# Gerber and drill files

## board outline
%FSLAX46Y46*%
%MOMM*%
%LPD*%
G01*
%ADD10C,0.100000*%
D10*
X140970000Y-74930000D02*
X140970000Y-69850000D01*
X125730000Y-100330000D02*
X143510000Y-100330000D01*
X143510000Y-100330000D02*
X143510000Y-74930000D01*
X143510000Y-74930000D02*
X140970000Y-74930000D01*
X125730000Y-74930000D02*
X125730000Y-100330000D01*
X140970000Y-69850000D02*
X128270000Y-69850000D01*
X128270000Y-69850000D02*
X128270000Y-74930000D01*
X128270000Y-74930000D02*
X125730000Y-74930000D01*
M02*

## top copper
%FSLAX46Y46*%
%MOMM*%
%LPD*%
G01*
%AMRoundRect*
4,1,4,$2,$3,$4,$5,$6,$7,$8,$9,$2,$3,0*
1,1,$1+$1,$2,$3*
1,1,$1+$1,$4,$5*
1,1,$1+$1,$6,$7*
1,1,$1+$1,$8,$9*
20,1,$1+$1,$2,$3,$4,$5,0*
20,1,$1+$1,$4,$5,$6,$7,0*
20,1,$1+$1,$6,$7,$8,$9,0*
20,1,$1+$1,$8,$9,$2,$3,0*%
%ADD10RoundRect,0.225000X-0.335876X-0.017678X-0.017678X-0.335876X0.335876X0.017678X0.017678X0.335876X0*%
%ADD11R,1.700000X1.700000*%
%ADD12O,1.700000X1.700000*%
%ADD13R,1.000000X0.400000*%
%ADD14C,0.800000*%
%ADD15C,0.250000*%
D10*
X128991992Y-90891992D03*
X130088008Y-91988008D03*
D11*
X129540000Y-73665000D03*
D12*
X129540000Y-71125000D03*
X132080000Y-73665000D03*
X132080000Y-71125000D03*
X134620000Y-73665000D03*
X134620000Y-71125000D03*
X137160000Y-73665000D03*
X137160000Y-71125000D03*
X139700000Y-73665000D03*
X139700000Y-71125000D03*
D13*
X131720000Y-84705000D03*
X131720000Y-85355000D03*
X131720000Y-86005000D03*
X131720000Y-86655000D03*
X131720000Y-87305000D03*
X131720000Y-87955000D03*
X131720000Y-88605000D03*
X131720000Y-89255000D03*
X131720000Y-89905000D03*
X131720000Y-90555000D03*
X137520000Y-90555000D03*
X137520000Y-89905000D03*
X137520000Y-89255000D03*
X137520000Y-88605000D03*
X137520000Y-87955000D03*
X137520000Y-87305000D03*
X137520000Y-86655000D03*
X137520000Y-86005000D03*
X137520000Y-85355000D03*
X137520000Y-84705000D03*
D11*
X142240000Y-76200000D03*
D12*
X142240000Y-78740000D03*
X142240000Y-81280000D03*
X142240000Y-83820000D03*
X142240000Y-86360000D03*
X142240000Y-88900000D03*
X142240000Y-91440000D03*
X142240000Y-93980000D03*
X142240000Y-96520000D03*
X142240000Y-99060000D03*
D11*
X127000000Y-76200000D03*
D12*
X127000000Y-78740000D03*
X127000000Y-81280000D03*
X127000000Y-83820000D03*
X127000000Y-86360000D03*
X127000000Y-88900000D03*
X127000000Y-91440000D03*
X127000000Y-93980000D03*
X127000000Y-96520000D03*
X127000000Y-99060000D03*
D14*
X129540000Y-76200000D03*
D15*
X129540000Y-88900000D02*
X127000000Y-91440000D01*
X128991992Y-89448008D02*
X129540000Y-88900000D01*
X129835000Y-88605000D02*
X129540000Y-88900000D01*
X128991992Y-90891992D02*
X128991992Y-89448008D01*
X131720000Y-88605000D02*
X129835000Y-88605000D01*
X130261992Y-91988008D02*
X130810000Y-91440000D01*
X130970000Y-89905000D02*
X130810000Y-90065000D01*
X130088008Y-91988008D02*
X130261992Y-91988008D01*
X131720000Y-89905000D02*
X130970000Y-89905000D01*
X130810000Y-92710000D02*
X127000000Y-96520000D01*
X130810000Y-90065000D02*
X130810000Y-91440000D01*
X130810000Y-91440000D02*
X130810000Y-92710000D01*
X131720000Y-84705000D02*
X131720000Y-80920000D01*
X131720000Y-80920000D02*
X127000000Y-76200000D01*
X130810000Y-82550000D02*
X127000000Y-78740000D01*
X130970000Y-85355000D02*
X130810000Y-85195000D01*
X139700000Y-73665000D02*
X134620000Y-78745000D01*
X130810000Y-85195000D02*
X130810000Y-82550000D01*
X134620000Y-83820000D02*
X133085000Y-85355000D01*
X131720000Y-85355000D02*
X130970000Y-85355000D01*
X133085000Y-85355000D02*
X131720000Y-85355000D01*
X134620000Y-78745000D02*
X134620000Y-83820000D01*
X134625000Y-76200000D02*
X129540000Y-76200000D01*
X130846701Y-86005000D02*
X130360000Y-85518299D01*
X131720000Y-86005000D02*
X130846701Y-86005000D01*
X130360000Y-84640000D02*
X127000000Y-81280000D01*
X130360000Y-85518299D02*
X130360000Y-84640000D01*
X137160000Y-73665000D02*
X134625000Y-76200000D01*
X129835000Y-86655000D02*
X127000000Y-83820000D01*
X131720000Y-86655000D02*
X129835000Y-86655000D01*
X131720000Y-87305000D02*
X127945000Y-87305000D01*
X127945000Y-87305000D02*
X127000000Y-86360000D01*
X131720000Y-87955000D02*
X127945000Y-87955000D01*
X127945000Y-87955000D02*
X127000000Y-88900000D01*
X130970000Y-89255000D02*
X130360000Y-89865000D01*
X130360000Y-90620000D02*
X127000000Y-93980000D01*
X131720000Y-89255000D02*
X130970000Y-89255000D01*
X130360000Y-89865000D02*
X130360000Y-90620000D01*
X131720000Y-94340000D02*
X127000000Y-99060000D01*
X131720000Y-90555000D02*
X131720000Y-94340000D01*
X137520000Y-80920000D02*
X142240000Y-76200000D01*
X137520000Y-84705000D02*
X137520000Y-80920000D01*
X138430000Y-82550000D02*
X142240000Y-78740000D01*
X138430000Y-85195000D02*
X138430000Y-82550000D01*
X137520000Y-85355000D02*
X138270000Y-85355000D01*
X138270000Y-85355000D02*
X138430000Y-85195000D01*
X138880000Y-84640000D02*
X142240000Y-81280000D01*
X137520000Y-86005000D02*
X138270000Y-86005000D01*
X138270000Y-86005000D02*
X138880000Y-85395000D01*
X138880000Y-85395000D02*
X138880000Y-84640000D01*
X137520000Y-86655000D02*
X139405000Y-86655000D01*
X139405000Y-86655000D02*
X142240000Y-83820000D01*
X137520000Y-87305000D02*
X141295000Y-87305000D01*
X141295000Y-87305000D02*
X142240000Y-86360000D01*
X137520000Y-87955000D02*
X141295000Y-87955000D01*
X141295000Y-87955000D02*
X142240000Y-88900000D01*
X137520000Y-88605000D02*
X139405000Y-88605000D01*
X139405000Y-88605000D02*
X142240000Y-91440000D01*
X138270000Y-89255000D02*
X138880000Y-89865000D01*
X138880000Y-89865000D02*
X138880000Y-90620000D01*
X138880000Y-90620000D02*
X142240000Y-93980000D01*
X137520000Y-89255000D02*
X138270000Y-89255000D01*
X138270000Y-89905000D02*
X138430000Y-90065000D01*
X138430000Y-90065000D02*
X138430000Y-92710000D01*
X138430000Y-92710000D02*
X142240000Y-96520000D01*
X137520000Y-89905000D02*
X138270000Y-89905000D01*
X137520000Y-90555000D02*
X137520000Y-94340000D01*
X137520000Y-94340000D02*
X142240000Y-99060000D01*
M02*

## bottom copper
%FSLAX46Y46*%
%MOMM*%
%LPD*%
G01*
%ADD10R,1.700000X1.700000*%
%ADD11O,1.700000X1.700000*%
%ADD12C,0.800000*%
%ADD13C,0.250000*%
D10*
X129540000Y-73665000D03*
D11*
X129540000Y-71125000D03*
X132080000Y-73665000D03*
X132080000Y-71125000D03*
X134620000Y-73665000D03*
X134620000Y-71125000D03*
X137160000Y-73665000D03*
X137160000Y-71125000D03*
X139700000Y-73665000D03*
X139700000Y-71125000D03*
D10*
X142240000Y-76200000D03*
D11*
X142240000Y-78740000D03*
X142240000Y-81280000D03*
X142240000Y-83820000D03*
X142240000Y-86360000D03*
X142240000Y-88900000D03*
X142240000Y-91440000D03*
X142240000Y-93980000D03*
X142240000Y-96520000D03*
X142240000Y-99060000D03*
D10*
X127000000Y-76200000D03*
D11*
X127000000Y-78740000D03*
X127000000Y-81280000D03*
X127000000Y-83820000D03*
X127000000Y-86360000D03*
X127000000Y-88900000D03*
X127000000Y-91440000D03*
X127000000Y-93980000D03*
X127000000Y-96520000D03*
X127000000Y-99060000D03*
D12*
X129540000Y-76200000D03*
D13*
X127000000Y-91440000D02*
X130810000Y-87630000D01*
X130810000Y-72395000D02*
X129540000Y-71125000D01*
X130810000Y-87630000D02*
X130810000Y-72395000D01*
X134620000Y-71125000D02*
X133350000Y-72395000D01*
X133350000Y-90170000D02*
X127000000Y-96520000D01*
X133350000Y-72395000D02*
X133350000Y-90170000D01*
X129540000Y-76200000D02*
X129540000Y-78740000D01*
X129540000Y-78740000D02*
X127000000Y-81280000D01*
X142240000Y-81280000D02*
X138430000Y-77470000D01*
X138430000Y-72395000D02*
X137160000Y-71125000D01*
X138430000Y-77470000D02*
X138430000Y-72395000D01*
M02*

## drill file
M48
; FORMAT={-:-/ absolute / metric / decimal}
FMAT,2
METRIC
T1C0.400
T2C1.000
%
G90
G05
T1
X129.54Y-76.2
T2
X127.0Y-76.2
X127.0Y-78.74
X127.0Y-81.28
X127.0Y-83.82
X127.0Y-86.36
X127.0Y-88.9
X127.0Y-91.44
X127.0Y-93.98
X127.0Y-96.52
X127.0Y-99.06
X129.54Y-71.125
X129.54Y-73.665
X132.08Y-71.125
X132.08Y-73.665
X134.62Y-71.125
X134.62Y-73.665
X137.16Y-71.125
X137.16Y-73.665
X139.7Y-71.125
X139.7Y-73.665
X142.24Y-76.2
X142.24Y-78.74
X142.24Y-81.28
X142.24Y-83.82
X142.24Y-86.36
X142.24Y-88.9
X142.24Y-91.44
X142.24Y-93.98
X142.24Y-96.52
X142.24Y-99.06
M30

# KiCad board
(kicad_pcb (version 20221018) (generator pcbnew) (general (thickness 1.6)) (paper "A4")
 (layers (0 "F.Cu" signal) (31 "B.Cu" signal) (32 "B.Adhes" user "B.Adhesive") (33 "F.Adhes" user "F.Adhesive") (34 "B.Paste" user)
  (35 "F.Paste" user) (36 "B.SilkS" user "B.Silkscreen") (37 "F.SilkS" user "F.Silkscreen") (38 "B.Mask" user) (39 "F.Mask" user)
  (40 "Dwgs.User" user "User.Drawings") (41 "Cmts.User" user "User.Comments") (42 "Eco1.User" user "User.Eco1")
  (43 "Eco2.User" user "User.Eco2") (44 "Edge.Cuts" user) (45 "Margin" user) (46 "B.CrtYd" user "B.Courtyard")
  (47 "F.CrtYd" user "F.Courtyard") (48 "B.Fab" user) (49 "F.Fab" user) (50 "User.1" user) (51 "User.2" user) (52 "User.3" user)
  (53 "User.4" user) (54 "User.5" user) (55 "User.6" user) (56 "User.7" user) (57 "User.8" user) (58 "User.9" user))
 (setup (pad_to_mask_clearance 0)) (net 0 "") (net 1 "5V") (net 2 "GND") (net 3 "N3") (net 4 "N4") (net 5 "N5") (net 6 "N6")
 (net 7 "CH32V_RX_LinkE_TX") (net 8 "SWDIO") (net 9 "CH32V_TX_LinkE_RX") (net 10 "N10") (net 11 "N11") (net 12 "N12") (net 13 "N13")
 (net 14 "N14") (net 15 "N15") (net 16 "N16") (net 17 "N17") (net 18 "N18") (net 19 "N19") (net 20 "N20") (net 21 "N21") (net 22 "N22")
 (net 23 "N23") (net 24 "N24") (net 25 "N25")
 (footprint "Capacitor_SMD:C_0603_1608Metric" (layer "F.Cu") (at 129.54 91.44 -45)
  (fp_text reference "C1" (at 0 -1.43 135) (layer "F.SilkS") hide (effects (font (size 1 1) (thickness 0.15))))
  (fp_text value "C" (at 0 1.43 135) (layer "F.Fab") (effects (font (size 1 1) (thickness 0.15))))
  (pad "1" smd roundrect (at -0.775 0 315) (size 0.9 0.95) (layers "F.Cu" "F.Paste" "F.Mask") (roundrect_rratio 0.25) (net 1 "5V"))
  (pad "2" smd roundrect (at 0.775 0 315) (size 0.9 0.95) (layers "F.Cu" "F.Paste" "F.Mask") (roundrect_rratio 0.25) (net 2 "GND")))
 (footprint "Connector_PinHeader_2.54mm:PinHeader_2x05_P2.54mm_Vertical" (layer "F.Cu") (at 129.54 73.665 90)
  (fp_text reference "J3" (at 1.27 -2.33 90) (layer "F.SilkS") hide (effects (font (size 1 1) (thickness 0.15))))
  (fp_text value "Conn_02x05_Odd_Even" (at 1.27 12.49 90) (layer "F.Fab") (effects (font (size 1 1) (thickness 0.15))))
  (pad "1" thru_hole rect (at 0 0 90) (size 1.7 1.7) (drill 1) (layers "*.Cu" "*.Mask") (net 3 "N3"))
  (pad "2" thru_hole oval (at 2.54 0 90) (size 1.7 1.7) (drill 1) (layers "*.Cu" "*.Mask") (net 1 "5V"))
  (pad "3" thru_hole oval (at 0 2.54 90) (size 1.7 1.7) (drill 1) (layers "*.Cu" "*.Mask") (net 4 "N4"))
  (pad "4" thru_hole oval (at 2.54 2.54 90) (size 1.7 1.7) (drill 1) (layers "*.Cu" "*.Mask") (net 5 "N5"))
  (pad "5" thru_hole oval (at 0 5.08 90) (size 1.7 1.7) (drill 1) (layers "*.Cu" "*.Mask") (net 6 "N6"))
  (pad "6" thru_hole oval (at 2.54 5.08 90) (size 1.7 1.7) (drill 1) (layers "*.Cu" "*.Mask") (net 2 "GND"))
  (pad "7" thru_hole oval (at 0 7.62 90) (size 1.7 1.7) (drill 1) (layers "*.Cu" "*.Mask") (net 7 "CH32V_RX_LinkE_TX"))
  (pad "8" thru_hole oval (at 2.54 7.62 90) (size 1.7 1.7) (drill 1) (layers "*.Cu" "*.Mask") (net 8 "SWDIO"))
  (pad "9" thru_hole oval (at 0 10.16 90) (size 1.7 1.7) (drill 1) (layers "*.Cu" "*.Mask") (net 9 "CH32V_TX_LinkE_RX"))
  (pad "10" thru_hole oval (at 2.54 10.16 90) (size 1.7 1.7) (drill 1) (layers "*.Cu" "*.Mask") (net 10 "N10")))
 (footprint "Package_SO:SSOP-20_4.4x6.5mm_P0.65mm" (layer "F.Cu") (at 134.62 87.63)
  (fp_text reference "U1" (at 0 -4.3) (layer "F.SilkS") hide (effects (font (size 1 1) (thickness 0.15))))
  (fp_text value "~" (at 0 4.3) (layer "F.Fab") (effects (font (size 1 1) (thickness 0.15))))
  (pad "1" smd rect (at -2.9 -2.925) (size 1 0.4) (layers "F.Cu" "F.Paste" "F.Mask") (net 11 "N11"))
  (pad "2" smd rect (at -2.9 -2.275) (size 1 0.4) (layers "F.Cu" "F.Paste" "F.Mask") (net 9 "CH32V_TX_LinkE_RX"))
  (pad "3" smd rect (at -2.9 -1.625) (size 1 0.4) (layers "F.Cu" "F.Paste" "F.Mask") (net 7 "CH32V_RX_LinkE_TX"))
  (pad "4" smd rect (at -2.9 -0.975) (size 1 0.4) (layers "F.Cu" "F.Paste" "F.Mask") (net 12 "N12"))
  (pad "5" smd rect (at -2.9 -0.325) (size 1 0.4) (layers "F.Cu" "F.Paste" "F.Mask") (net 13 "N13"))
  (pad "6" smd rect (at -2.9 0.325) (size 1 0.4) (layers "F.Cu" "F.Paste" "F.Mask") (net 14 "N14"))
  (pad "7" smd rect (at -2.9 0.975) (size 1 0.4) (layers "F.Cu" "F.Paste" "F.Mask") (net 1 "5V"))
  (pad "8" smd rect (at -2.9 1.625) (size 1 0.4) (layers "F.Cu" "F.Paste" "F.Mask") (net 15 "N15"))
  (pad "9" smd rect (at -2.9 2.275) (size 1 0.4) (layers "F.Cu" "F.Paste" "F.Mask") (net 2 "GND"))
  (pad "10" smd rect (at -2.9 2.925) (size 1 0.4) (layers "F.Cu" "F.Paste" "F.Mask") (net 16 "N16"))
  (pad "11" smd rect (at 2.9 2.925) (size 1 0.4) (layers "F.Cu" "F.Paste" "F.Mask") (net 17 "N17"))
  (pad "12" smd rect (at 2.9 2.275) (size 1 0.4) (layers "F.Cu" "F.Paste" "F.Mask") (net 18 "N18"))
  (pad "13" smd rect (at 2.9 1.625) (size 1 0.4) (layers "F.Cu" "F.Paste" "F.Mask") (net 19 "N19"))
  (pad "14" smd rect (at 2.9 0.975) (size 1 0.4) (layers "F.Cu" "F.Paste" "F.Mask") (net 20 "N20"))
  (pad "15" smd rect (at 2.9 0.325) (size 1 0.4) (layers "F.Cu" "F.Paste" "F.Mask") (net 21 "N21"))
  (pad "16" smd rect (at 2.9 -0.325) (size 1 0.4) (layers "F.Cu" "F.Paste" "F.Mask") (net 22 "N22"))
  (pad "17" smd rect (at 2.9 -0.975) (size 1 0.4) (layers "F.Cu" "F.Paste" "F.Mask") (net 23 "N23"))
  (pad "18" smd rect (at 2.9 -1.625) (size 1 0.4) (layers "F.Cu" "F.Paste" "F.Mask") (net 8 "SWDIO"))
  (pad "19" smd rect (at 2.9 -2.275) (size 1 0.4) (layers "F.Cu" "F.Paste" "F.Mask") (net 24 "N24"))
  (pad "20" smd rect (at 2.9 -2.925) (size 1 0.4) (layers "F.Cu" "F.Paste" "F.Mask") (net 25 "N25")))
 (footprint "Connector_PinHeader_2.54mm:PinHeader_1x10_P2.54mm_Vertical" (layer "B.Cu") (at 142.24 76.2 180)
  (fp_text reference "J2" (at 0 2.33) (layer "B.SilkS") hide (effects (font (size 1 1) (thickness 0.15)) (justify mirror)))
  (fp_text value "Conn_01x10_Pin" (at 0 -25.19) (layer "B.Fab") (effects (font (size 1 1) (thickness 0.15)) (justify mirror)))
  (pad "1" thru_hole rect (at 0 0 180) (size 1.7 1.7) (drill 1) (layers "*.Cu" "*.Mask") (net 25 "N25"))
  (pad "2" thru_hole oval (at 0 -2.54 180) (size 1.7 1.7) (drill 1) (layers "*.Cu" "*.Mask") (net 24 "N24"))
  (pad "3" thru_hole oval (at 0 -5.08 180) (size 1.7 1.7) (drill 1) (layers "*.Cu" "*.Mask") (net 8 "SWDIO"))
  (pad "4" thru_hole oval (at 0 -7.62 180) (size 1.7 1.7) (drill 1) (layers "*.Cu" "*.Mask") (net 23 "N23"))
  (pad "5" thru_hole oval (at 0 -10.16 180) (size 1.7 1.7) (drill 1) (layers "*.Cu" "*.Mask") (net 22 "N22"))
  (pad "6" thru_hole oval (at 0 -12.7 180) (size 1.7 1.7) (drill 1) (layers "*.Cu" "*.Mask") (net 21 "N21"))
  (pad "7" thru_hole oval (at 0 -15.24 180) (size 1.7 1.7) (drill 1) (layers "*.Cu" "*.Mask") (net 20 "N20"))
  (pad "8" thru_hole oval (at 0 -17.78 180) (size 1.7 1.7) (drill 1) (layers "*.Cu" "*.Mask") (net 19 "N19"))
  (pad "9" thru_hole oval (at 0 -20.32 180) (size 1.7 1.7) (drill 1) (layers "*.Cu" "*.Mask") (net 18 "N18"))
  (pad "10" thru_hole oval (at 0 -22.86 180) (size 1.7 1.7) (drill 1) (layers "*.Cu" "*.Mask") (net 17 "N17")))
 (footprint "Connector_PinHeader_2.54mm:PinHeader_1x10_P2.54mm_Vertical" (layer "B.Cu") (at 127 76.2 180)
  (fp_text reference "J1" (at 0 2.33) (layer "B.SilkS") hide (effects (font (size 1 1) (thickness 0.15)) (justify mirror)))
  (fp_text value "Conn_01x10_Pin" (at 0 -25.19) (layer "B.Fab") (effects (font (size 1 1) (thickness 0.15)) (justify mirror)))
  (pad "1" thru_hole rect (at 0 0 180) (size 1.7 1.7) (drill 1) (layers "*.Cu" "*.Mask") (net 11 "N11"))
  (pad "2" thru_hole oval (at 0 -2.54 180) (size 1.7 1.7) (drill 1) (layers "*.Cu" "*.Mask") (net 9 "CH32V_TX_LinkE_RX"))
  (pad "3" thru_hole oval (at 0 -5.08 180) (size 1.7 1.7) (drill 1) (layers "*.Cu" "*.Mask") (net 7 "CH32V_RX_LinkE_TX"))
  (pad "4" thru_hole oval (at 0 -7.62 180) (size 1.7 1.7) (drill 1) (layers "*.Cu" "*.Mask") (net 12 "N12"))
  (pad "5" thru_hole oval (at 0 -10.16 180) (size 1.7 1.7) (drill 1) (layers "*.Cu" "*.Mask") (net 13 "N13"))
  (pad "6" thru_hole oval (at 0 -12.7 180) (size 1.7 1.7) (drill 1) (layers "*.Cu" "*.Mask") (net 14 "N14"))
  (pad "7" thru_hole oval (at 0 -15.24 180) (size 1.7 1.7) (drill 1) (layers "*.Cu" "*.Mask") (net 1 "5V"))
  (pad "8" thru_hole oval (at 0 -17.78 180) (size 1.7 1.7) (drill 1) (layers "*.Cu" "*.Mask") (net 15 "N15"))
  (pad "9" thru_hole oval (at 0 -20.32 180) (size 1.7 1.7) (drill 1) (layers "*.Cu" "*.Mask") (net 2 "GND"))
  (pad "10" thru_hole oval (at 0 -22.86 180) (size 1.7 1.7) (drill 1) (layers "*.Cu" "*.Mask") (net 16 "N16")))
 (gr_line (start 140.97 74.93) (end 140.97 69.85) (stroke (width 0.1) (type default)) (layer "Edge.Cuts"))
 (gr_line (start 125.73 100.33) (end 143.51 100.33) (stroke (width 0.1) (type default)) (layer "Edge.Cuts"))
 (gr_line (start 143.51 100.33) (end 143.51 74.93) (stroke (width 0.1) (type default)) (layer "Edge.Cuts"))
 (gr_line (start 143.51 74.93) (end 140.97 74.93) (stroke (width 0.1) (type default)) (layer "Edge.Cuts"))
 (gr_line (start 125.73 74.93) (end 125.73 100.33) (stroke (width 0.1) (type default)) (layer "Edge.Cuts"))
 (gr_line (start 140.97 69.85) (end 128.27 69.85) (stroke (width 0.1) (type default)) (layer "Edge.Cuts"))
 (gr_line (start 128.27 69.85) (end 128.27 74.93) (stroke (width 0.1) (type default)) (layer "Edge.Cuts"))
 (gr_line (start 128.27 74.93) (end 125.73 74.93) (stroke (width 0.1) (type default)) (layer "Edge.Cuts"))
 (segment (start 129.54 88.9) (end 127 91.44) (width 0.25) (layer "F.Cu") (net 1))
 (segment (start 128.991992 89.448008) (end 129.54 88.9) (width 0.25) (layer "F.Cu") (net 1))
 (segment (start 129.835 88.605) (end 129.54 88.9) (width 0.25) (layer "F.Cu") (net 1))
 (segment (start 128.991992 90.891992) (end 128.991992 89.448008) (width 0.25) (layer "F.Cu") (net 1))
 (segment (start 131.72 88.605) (end 129.835 88.605) (width 0.25) (layer "F.Cu") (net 1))
 (segment (start 127 91.44) (end 130.81 87.63) (width 0.25) (layer "B.Cu") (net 1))
 (segment (start 130.81 72.395) (end 129.54 71.125) (width 0.25) (layer "B.Cu") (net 1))
 (segment (start 130.81 87.63) (end 130.81 72.395) (width 0.25) (layer "B.Cu") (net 1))
 (segment (start 130.261992 91.988008) (end 130.81 91.44) (width 0.25) (layer "F.Cu") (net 2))
 (segment (start 130.97 89.905) (end 130.81 90.065) (width 0.25) (layer "F.Cu") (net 2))
 (segment (start 130.088008 91.988008) (end 130.261992 91.988008) (width 0.25) (layer "F.Cu") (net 2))
 (segment (start 131.72 89.905) (end 130.97 89.905) (width 0.25) (layer "F.Cu") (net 2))
 (segment (start 130.81 92.71) (end 127 96.52) (width 0.25) (layer "F.Cu") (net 2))
 (segment (start 130.81 90.065) (end 130.81 91.44) (width 0.25) (layer "F.Cu") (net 2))
 (segment (start 130.81 91.44) (end 130.81 92.71) (width 0.25) (layer "F.Cu") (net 2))
 (segment (start 134.62 71.125) (end 133.35 72.395) (width 0.25) (layer "B.Cu") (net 2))
 (segment (start 133.35 90.17) (end 127 96.52) (width 0.25) (layer "B.Cu") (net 2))
 (segment (start 133.35 72.395) (end 133.35 90.17) (width 0.25) (layer "B.Cu") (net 2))
 (segment (start 131.72 84.705) (end 131.72 80.92) (width 0.25) (layer "F.Cu") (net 11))
 (segment (start 131.72 80.92) (end 127 76.2) (width 0.25) (layer "F.Cu") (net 11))
 (segment (start 130.81 82.55) (end 127 78.74) (width 0.25) (layer "F.Cu") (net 9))
 (segment (start 130.97 85.355) (end 130.81 85.195) (width 0.25) (layer "F.Cu") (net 9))
 (segment (start 139.7 73.665) (end 134.62 78.745) (width 0.25) (layer "F.Cu") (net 9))
 (segment (start 130.81 85.195) (end 130.81 82.55) (width 0.25) (layer "F.Cu") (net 9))
 (segment (start 134.62 83.82) (end 133.085 85.355) (width 0.25) (layer "F.Cu") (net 9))
 (segment (start 131.72 85.355) (end 130.97 85.355) (width 0.25) (layer "F.Cu") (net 9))
 (segment (start 133.085 85.355) (end 131.72 85.355) (width 0.25) (layer "F.Cu") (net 9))
 (segment (start 134.62 78.745) (end 134.62 83.82) (width 0.25) (layer "F.Cu") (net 9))
 (segment (start 134.625 76.2) (end 129.54 76.2) (width 0.25) (layer "F.Cu") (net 7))
 (segment (start 130.846701 86.005) (end 130.36 85.518299) (width 0.25) (layer "F.Cu") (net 7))
 (segment (start 131.72 86.005) (end 130.846701 86.005) (width 0.25) (layer "F.Cu") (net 7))
 (segment (start 130.36 84.64) (end 127 81.28) (width 0.25) (layer "F.Cu") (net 7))
 (segment (start 130.36 85.518299) (end 130.36 84.64) (width 0.25) (layer "F.Cu") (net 7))
 (segment (start 137.16 73.665) (end 134.625 76.2) (width 0.25) (layer "F.Cu") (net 7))
 (via (at 129.54 76.2) (size 0.8) (drill 0.4) (layers "F.Cu" "B.Cu") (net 7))
 (segment (start 129.54 76.2) (end 129.54 78.74) (width 0.25) (layer "B.Cu") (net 7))
 (segment (start 129.54 78.74) (end 127 81.28) (width 0.25) (layer "B.Cu") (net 7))
 (segment (start 129.835 86.655) (end 127 83.82) (width 0.25) (layer "F.Cu") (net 12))
 (segment (start 131.72 86.655) (end 129.835 86.655) (width 0.25) (layer "F.Cu") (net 12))
 (segment (start 131.72 87.305) (end 127.945 87.305) (width 0.25) (layer "F.Cu") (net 13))
 (segment (start 127.945 87.305) (end 127 86.36) (width 0.25) (layer "F.Cu") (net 13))
 (segment (start 131.72 87.955) (end 127.945 87.955) (width 0.25) (layer "F.Cu") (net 14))
 (segment (start 127.945 87.955) (end 127 88.9) (width 0.25) (layer "F.Cu") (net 14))
 (segment (start 130.97 89.255) (end 130.36 89.865) (width 0.25) (layer "F.Cu") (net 15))
 (segment (start 130.36 90.62) (end 127 93.98) (width 0.25) (layer "F.Cu") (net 15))
 (segment (start 131.72 89.255) (end 130.97 89.255) (width 0.25) (layer "F.Cu") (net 15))
 (segment (start 130.36 89.865) (end 130.36 90.62) (width 0.25) (layer "F.Cu") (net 15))
 (segment (start 131.72 94.34) (end 127 99.06) (width 0.25) (layer "F.Cu") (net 16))
 (segment (start 131.72 90.555) (end 131.72 94.34) (width 0.25) (layer "F.Cu") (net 16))
 (segment (start 137.52 80.92) (end 142.24 76.2) (width 0.25) (layer "F.Cu") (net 25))
 (segment (start 137.52 84.705) (end 137.52 80.92) (width 0.25) (layer "F.Cu") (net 25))
 (segment (start 138.43 82.55) (end 142.24 78.74) (width 0.25) (layer "F.Cu") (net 24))
 (segment (start 138.43 85.195) (end 138.43 82.55) (width 0.25) (layer "F.Cu") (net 24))
 (segment (start 137.52 85.355) (end 138.27 85.355) (width 0.25) (layer "F.Cu") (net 24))
 (segment (start 138.27 85.355) (end 138.43 85.195) (width 0.25) (layer "F.Cu") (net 24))
 (segment (start 138.88 84.64) (end 142.24 81.28) (width 0.25) (layer "F.Cu") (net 8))
 (segment (start 137.52 86.005) (end 138.27 86.005) (width 0.25) (layer "F.Cu") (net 8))
 (segment (start 138.27 86.005) (end 138.88 85.395) (width 0.25) (layer "F.Cu") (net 8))
 (segment (start 138.88 85.395) (end 138.88 84.64) (width 0.25) (layer "F.Cu") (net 8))
 (segment (start 142.24 81.28) (end 138.43 77.47) (width 0.25) (layer "B.Cu") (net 8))
 (segment (start 138.43 72.395) (end 137.16 71.125) (width 0.25) (layer "B.Cu") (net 8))
 (segment (start 138.43 77.47) (end 138.43 72.395) (width 0.25) (layer "B.Cu") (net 8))
 (segment (start 137.52 86.655) (end 139.405 86.655) (width 0.25) (layer "F.Cu") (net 23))
 (segment (start 139.405 86.655) (end 142.24 83.82) (width 0.25) (layer "F.Cu") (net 23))
 (segment (start 137.52 87.305) (end 141.295 87.305) (width 0.25) (layer "F.Cu") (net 22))
 (segment (start 141.295 87.305) (end 142.24 86.36) (width 0.25) (layer "F.Cu") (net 22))
 (segment (start 137.52 87.955) (end 141.295 87.955) (width 0.25) (layer "F.Cu") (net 21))
 (segment (start 141.295 87.955) (end 142.24 88.9) (width 0.25) (layer "F.Cu") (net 21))
 (segment (start 137.52 88.605) (end 139.405 88.605) (width 0.25) (layer "F.Cu") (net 20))
 (segment (start 139.405 88.605) (end 142.24 91.44) (width 0.25) (layer "F.Cu") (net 20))
 (segment (start 138.27 89.255) (end 138.88 89.865) (width 0.25) (layer "F.Cu") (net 19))
 (segment (start 138.88 89.865) (end 138.88 90.62) (width 0.25) (layer "F.Cu") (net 19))
 (segment (start 138.88 90.62) (end 142.24 93.98) (width 0.25) (layer "F.Cu") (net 19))
 (segment (start 137.52 89.255) (end 138.27 89.255) (width 0.25) (layer "F.Cu") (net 19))
 (segment (start 138.27 89.905) (end 138.43 90.065) (width 0.25) (layer "F.Cu") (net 18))
 (segment (start 138.43 90.065) (end 138.43 92.71) (width 0.25) (layer "F.Cu") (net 18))
 (segment (start 138.43 92.71) (end 142.24 96.52) (width 0.25) (layer "F.Cu") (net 18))
 (segment (start 137.52 89.905) (end 138.27 89.905) (width 0.25) (layer "F.Cu") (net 18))
 (segment (start 137.52 90.555) (end 137.52 94.34) (width 0.25) (layer "F.Cu") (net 17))
 (segment (start 137.52 94.34) (end 142.24 99.06) (width 0.25) (layer "F.Cu") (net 17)))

